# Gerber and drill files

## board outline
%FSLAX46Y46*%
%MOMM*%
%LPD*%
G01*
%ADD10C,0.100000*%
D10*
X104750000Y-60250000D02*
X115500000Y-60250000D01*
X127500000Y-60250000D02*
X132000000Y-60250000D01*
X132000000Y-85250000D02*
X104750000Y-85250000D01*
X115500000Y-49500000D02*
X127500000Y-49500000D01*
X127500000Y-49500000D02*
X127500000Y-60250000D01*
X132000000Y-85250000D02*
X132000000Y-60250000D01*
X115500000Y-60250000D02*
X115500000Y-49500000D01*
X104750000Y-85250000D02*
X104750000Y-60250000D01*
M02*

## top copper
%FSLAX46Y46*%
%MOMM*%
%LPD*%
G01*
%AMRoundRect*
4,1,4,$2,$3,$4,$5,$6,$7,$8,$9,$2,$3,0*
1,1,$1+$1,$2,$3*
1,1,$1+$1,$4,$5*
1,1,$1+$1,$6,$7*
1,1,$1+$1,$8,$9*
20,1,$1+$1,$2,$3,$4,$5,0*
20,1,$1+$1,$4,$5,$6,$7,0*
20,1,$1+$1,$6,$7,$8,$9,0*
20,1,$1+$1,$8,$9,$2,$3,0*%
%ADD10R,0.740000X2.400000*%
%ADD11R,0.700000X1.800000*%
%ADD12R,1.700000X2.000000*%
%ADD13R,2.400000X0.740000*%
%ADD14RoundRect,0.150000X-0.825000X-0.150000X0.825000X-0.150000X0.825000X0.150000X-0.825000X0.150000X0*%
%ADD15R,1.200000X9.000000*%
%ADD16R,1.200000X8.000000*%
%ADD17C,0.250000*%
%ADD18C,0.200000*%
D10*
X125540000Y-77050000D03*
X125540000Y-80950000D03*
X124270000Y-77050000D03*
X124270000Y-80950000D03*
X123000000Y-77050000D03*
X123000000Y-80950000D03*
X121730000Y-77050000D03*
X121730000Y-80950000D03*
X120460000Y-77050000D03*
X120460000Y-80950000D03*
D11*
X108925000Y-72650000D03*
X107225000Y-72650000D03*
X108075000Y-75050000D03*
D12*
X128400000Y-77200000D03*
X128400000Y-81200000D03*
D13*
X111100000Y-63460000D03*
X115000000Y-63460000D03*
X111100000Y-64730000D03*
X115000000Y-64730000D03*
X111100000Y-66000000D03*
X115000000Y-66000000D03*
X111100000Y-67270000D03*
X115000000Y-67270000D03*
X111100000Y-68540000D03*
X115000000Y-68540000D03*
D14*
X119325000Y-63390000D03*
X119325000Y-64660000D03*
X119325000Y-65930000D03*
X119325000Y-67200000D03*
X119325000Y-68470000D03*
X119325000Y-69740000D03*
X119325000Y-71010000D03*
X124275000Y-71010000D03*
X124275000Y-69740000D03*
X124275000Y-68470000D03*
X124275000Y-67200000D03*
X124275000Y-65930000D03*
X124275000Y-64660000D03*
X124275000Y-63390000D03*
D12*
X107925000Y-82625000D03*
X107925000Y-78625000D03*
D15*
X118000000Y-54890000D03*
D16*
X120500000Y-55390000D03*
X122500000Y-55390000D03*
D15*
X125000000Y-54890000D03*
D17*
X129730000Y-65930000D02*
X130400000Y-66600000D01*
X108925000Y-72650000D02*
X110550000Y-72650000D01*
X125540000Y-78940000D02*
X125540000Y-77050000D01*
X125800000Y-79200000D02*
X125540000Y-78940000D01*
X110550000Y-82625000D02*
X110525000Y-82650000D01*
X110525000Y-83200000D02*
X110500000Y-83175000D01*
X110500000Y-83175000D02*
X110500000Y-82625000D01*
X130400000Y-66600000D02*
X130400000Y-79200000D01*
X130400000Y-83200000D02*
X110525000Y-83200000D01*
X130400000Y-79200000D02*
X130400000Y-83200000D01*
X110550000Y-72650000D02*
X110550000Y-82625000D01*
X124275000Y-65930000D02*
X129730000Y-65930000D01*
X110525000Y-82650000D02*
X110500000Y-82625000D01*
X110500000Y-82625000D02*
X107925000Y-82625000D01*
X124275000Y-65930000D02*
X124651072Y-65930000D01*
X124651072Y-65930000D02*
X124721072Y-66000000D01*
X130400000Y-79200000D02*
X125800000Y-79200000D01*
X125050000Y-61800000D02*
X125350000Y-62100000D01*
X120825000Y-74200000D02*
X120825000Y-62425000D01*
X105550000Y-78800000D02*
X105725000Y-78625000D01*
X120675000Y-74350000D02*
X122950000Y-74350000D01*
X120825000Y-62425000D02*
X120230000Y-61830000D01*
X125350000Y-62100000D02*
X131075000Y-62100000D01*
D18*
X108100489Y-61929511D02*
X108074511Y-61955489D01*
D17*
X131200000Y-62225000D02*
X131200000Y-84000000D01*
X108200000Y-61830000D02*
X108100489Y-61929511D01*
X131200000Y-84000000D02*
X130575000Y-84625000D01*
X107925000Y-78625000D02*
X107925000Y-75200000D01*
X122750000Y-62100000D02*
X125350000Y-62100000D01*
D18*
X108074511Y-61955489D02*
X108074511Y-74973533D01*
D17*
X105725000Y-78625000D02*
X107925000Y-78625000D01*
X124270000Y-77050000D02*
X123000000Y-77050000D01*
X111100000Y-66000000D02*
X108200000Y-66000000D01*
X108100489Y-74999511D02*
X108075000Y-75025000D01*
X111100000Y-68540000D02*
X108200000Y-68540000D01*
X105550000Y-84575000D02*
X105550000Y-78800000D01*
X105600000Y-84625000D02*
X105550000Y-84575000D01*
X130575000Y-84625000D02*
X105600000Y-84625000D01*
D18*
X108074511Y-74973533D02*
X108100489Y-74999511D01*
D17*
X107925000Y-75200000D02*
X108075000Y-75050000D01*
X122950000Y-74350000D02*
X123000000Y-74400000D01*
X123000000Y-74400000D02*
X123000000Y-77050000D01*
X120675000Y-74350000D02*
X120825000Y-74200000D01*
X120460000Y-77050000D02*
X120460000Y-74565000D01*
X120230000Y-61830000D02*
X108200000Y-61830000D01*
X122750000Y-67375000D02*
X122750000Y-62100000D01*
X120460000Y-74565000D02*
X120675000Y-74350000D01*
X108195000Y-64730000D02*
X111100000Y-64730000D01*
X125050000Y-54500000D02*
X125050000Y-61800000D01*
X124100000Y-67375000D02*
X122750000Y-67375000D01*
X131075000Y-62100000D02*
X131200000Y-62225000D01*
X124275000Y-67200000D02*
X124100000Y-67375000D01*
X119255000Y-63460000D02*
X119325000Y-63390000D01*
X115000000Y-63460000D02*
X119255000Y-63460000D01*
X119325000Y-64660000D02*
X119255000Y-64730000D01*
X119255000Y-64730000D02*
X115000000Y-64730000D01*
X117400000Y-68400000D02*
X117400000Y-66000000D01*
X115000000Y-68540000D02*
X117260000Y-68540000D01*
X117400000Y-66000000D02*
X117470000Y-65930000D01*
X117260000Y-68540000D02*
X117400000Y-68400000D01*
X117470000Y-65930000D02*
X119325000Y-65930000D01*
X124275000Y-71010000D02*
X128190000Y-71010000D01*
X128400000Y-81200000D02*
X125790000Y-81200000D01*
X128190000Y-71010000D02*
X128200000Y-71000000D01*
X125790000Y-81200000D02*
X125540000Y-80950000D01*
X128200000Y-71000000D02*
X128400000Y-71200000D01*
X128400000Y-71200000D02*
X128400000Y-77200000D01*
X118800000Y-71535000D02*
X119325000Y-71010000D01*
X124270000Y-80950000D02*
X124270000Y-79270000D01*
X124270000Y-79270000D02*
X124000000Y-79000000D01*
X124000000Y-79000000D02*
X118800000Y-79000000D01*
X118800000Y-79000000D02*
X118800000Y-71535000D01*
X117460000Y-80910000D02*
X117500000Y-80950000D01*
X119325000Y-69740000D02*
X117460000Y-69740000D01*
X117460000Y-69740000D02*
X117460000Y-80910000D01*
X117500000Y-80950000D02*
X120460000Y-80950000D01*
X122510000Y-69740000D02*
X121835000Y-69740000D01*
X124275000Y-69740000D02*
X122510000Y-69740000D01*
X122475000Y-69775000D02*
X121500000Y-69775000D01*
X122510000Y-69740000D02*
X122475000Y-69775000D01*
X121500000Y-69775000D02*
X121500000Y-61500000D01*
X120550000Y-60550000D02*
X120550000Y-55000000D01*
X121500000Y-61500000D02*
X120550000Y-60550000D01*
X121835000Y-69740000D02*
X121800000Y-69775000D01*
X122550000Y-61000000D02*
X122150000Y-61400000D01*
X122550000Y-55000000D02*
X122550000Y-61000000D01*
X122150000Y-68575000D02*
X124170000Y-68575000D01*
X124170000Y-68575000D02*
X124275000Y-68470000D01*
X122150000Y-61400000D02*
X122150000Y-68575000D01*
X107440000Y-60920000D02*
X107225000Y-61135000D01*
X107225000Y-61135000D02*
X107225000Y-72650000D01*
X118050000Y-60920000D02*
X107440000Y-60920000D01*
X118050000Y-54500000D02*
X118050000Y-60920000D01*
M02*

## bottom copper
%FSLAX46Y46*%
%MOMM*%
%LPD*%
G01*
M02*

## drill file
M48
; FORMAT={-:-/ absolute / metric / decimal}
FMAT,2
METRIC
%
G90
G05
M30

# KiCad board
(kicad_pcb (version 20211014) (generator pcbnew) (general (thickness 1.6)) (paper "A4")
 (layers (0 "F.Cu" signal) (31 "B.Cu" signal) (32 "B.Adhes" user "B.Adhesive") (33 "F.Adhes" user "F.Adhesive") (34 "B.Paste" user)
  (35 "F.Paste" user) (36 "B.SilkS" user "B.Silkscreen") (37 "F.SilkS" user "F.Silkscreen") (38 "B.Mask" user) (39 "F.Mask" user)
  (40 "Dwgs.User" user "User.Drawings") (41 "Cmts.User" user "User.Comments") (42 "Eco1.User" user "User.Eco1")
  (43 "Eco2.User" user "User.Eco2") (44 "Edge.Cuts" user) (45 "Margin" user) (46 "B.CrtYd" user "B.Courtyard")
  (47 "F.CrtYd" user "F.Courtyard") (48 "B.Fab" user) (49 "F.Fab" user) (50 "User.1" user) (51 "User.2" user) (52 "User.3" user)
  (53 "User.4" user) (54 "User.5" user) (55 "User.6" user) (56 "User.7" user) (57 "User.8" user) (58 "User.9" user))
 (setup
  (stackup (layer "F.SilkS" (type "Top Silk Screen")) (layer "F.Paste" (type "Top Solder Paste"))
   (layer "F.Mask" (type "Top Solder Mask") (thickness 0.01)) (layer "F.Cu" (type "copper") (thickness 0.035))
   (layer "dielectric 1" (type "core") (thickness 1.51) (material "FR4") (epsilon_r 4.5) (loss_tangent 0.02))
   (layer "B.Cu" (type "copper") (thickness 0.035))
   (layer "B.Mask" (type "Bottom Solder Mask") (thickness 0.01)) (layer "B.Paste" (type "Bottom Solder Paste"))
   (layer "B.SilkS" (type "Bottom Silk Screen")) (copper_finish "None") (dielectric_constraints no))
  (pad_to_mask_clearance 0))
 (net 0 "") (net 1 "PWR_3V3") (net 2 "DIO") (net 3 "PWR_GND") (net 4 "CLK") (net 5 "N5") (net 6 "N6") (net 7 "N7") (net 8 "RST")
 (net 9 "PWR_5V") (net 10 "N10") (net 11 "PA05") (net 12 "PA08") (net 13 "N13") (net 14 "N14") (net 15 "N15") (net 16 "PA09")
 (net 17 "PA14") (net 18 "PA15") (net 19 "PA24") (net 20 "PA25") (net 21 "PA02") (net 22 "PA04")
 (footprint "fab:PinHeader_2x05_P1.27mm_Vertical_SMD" (layer "F.Cu") (at 123 79 -90)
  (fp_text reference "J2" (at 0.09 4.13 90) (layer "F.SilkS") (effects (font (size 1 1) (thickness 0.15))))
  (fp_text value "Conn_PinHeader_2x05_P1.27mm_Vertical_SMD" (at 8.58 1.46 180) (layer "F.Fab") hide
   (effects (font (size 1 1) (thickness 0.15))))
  (pad "1" smd rect locked (at -1.95 -2.54 270) (size 2.4 0.74) (layers "F.Cu" "F.Paste" "F.Mask") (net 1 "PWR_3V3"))
  (pad "2" smd rect locked (at 1.95 -2.54 270) (size 2.4 0.74) (layers "F.Cu" "F.Paste" "F.Mask") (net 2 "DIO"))
  (pad "3" smd rect locked (at -1.95 -1.27 270) (size 2.4 0.74) (layers "F.Cu" "F.Paste" "F.Mask") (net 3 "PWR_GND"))
  (pad "4" smd rect locked (at 1.95 -1.27 270) (size 2.4 0.74) (layers "F.Cu" "F.Paste" "F.Mask") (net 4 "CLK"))
  (pad "5" smd rect locked (at -1.95 0 270) (size 2.4 0.74) (layers "F.Cu" "F.Paste" "F.Mask") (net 3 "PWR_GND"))
  (pad "6" smd rect locked (at 1.95 0 270) (size 2.4 0.74) (layers "F.Cu" "F.Paste" "F.Mask") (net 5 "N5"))
  (pad "7" smd rect locked (at -1.95 1.27 270) (size 2.4 0.74) (layers "F.Cu" "F.Paste" "F.Mask") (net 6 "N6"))
  (pad "8" smd rect locked (at 1.95 1.27 270) (size 2.4 0.74) (layers "F.Cu" "F.Paste" "F.Mask") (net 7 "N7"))
  (pad "9" smd rect locked (at -1.95 2.54 270) (size 2.4 0.74) (layers "F.Cu" "F.Paste" "F.Mask") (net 3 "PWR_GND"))
  (pad "10" smd rect locked (at 1.95 2.54 270) (size 2.4 0.74) (layers "F.Cu" "F.Paste" "F.Mask") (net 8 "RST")))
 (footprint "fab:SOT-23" (layer "F.Cu") (at 108.075 73.85 -90)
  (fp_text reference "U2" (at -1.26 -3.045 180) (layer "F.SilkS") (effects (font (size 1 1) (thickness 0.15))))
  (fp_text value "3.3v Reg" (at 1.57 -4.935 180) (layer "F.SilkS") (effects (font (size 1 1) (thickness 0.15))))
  (pad "1" smd rect (at -1.2 -0.85 270) (size 1.8 0.7) (layers "F.Cu" "F.Paste" "F.Mask") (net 1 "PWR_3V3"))
  (pad "2" smd rect (at -1.2 0.85 270) (size 1.8 0.7) (layers "F.Cu" "F.Paste" "F.Mask") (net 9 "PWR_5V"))
  (pad "3" smd rect (at 1.2 0 270) (size 1.8 0.7) (layers "F.Cu" "F.Paste" "F.Mask") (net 3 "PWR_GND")))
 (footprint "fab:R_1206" (layer "F.Cu") (at 128.4 79.2 -90)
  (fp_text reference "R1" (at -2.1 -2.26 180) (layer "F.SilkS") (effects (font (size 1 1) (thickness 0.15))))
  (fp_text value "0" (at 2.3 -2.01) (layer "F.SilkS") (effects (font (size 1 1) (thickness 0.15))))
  (pad "1" smd rect locked (at -2 0 270) (size 2 1.7) (layers "F.Cu" "F.Paste" "F.Mask") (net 2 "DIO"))
  (pad "2" smd rect locked (at 2 0 270) (size 2 1.7) (layers "F.Cu" "F.Paste" "F.Mask") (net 2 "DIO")))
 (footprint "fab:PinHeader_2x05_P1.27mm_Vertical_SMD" (layer "F.Cu") (at 113.05 66)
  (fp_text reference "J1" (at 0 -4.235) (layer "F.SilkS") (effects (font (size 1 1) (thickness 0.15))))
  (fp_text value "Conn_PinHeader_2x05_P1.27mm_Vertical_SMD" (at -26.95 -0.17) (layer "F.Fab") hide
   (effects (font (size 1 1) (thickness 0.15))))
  (pad "1" smd rect locked (at -1.95 -2.54) (size 2.4 0.74) (layers "F.Cu" "F.Paste" "F.Mask") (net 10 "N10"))
  (pad "2" smd rect locked (at 1.95 -2.54) (size 2.4 0.74) (layers "F.Cu" "F.Paste" "F.Mask") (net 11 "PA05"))
  (pad "3" smd rect locked (at -1.95 -1.27) (size 2.4 0.74) (layers "F.Cu" "F.Paste" "F.Mask") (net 3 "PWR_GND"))
  (pad "4" smd rect locked (at 1.95 -1.27) (size 2.4 0.74) (layers "F.Cu" "F.Paste" "F.Mask") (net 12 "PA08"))
  (pad "5" smd rect locked (at -1.95 0) (size 2.4 0.74) (layers "F.Cu" "F.Paste" "F.Mask") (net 3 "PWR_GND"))
  (pad "6" smd rect locked (at 1.95 0) (size 2.4 0.74) (layers "F.Cu" "F.Paste" "F.Mask") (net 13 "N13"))
  (pad "7" smd rect locked (at -1.95 1.27) (size 2.4 0.74) (layers "F.Cu" "F.Paste" "F.Mask") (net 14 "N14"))
  (pad "8" smd rect locked (at 1.95 1.27) (size 2.4 0.74) (layers "F.Cu" "F.Paste" "F.Mask") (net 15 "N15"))
  (pad "9" smd rect locked (at -1.95 2.54) (size 2.4 0.74) (layers "F.Cu" "F.Paste" "F.Mask") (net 3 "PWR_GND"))
  (pad "10" smd rect locked (at 1.95 2.54) (size 2.4 0.74) (layers "F.Cu" "F.Paste" "F.Mask") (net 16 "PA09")))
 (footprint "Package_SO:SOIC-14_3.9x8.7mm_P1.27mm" (layer "F.Cu") (at 121.8 67.2)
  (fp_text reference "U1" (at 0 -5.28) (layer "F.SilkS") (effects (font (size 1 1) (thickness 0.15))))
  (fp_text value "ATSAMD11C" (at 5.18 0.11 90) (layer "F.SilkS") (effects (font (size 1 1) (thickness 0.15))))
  (pad "1" smd roundrect (at -2.475 -3.81) (size 1.95 0.6) (layers "F.Cu" "F.Paste" "F.Mask") (roundrect_rratio 0.25) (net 11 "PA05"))
  (pad "2" smd roundrect (at -2.475 -2.54) (size 1.95 0.6) (layers "F.Cu" "F.Paste" "F.Mask") (roundrect_rratio 0.25) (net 12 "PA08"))
  (pad "3" smd roundrect (at -2.475 -1.27) (size 1.95 0.6) (layers "F.Cu" "F.Paste" "F.Mask") (roundrect_rratio 0.25) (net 16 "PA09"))
  (pad "4" smd roundrect (at -2.475 0) (size 1.95 0.6) (layers "F.Cu" "F.Paste" "F.Mask") (roundrect_rratio 0.25) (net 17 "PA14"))
  (pad "5" smd roundrect (at -2.475 1.27) (size 1.95 0.6) (layers "F.Cu" "F.Paste" "F.Mask") (roundrect_rratio 0.25) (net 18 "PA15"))
  (pad "6" smd roundrect (at -2.475 2.54) (size 1.95 0.6) (layers "F.Cu" "F.Paste" "F.Mask") (roundrect_rratio 0.25) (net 8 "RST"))
  (pad "7" smd roundrect (at -2.475 3.81) (size 1.95 0.6) (layers "F.Cu" "F.Paste" "F.Mask") (roundrect_rratio 0.25) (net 4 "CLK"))
  (pad "8" smd roundrect (at 2.475 3.81) (size 1.95 0.6) (layers "F.Cu" "F.Paste" "F.Mask") (roundrect_rratio 0.25) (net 2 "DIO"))
  (pad "9" smd roundrect (at 2.475 2.54) (size 1.95 0.6) (layers "F.Cu" "F.Paste" "F.Mask") (roundrect_rratio 0.25) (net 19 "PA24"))
  (pad "10" smd roundrect (at 2.475 1.27) (size 1.95 0.6) (layers "F.Cu" "F.Paste" "F.Mask") (roundrect_rratio 0.25) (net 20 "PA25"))
  (pad "11" smd roundrect (at 2.475 0) (size 1.95 0.6) (layers "F.Cu" "F.Paste" "F.Mask") (roundrect_rratio 0.25) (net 3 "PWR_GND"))
  (pad "12" smd roundrect (at 2.475 -1.27) (size 1.95 0.6) (layers "F.Cu" "F.Paste" "F.Mask") (roundrect_rratio 0.25) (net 1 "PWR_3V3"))
  (pad "13" smd roundrect (at 2.475 -2.54) (size 1.95 0.6) (layers "F.Cu" "F.Paste" "F.Mask") (roundrect_rratio 0.25) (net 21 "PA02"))
  (pad "14" smd roundrect (at 2.475 -3.81) (size 1.95 0.6) (layers "F.Cu" "F.Paste" "F.Mask") (roundrect_rratio 0.25) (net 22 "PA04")))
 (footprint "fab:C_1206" (layer "F.Cu") (at 107.925 80.625 90)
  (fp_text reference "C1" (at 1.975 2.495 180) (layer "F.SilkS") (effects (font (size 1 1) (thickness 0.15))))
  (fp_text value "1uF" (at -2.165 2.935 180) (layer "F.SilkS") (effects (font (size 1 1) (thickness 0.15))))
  (pad "1" smd rect (at -2 0 90) (size 2 1.7) (layers "F.Cu" "F.Paste" "F.Mask") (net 1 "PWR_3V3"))
  (pad "2" smd rect (at 2 0 90) (size 2 1.7) (layers "F.Cu" "F.Paste" "F.Mask") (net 3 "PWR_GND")))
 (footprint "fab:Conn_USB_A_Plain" (layer "F.Cu") (at 121.5 54.89 90)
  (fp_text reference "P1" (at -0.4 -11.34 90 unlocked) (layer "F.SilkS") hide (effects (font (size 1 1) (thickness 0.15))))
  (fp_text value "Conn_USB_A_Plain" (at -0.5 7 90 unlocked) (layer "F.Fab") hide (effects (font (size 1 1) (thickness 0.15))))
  (pad "1" smd rect (at 0 -3.5 90) (size 9 1.2) (layers "F.Cu" "F.Paste" "F.Mask") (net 9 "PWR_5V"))
  (pad "2" smd rect (at -0.5 -1 90) (size 8 1.2) (layers "F.Cu" "F.Paste" "F.Mask") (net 19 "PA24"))
  (pad "3" smd rect (at -0.5 1 90) (size 8 1.2) (layers "F.Cu" "F.Paste" "F.Mask") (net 20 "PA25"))
  (pad "4" smd rect (at 0 3.5 90) (size 9 1.2) (layers "F.Cu" "F.Paste" "F.Mask") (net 3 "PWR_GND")))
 (gr_line (start 104.75 60.25) (end 115.5 60.25) (layer "Edge.Cuts") (width 0.1))
 (gr_line (start 127.5 60.25) (end 132 60.25) (layer "Edge.Cuts") (width 0.1))
 (gr_line (start 132 85.25) (end 104.75 85.25) (layer "Edge.Cuts") (width 0.1))
 (gr_line (start 115.5 49.5) (end 127.5 49.5) (layer "Edge.Cuts") (width 0.1))
 (gr_line (start 127.5 49.5) (end 127.5 60.25) (layer "Edge.Cuts") (width 0.1))
 (gr_line (start 132 85.25) (end 132 60.25) (layer "Edge.Cuts") (width 0.1))
 (gr_line (start 115.5 60.25) (end 115.5 49.5) (layer "Edge.Cuts") (width 0.1))
 (gr_line (start 104.75 85.25) (end 104.75 60.25) (layer "Edge.Cuts") (width 0.1))
 (segment (start 129.73 65.93) (end 130.4 66.6) (width 0.25) (layer "F.Cu") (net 1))
 (segment (start 108.925 72.65) (end 110.55 72.65) (width 0.25) (layer "F.Cu") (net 1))
 (segment (start 125.54 78.94) (end 125.54 77.05) (width 0.25) (layer "F.Cu") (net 1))
 (segment (start 125.8 79.2) (end 125.54 78.94) (width 0.25) (layer "F.Cu") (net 1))
 (segment (start 110.55 82.625) (end 110.525 82.65) (width 0.25) (layer "F.Cu") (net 1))
 (segment (start 110.525 83.2) (end 110.5 83.175) (width 0.25) (layer "F.Cu") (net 1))
 (segment (start 110.5 83.175) (end 110.5 82.625) (width 0.25) (layer "F.Cu") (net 1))
 (segment (start 130.4 66.6) (end 130.4 79.2) (width 0.25) (layer "F.Cu") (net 1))
 (segment (start 130.4 83.2) (end 110.525 83.2) (width 0.25) (layer "F.Cu") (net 1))
 (segment (start 130.4 79.2) (end 130.4 83.2) (width 0.25) (layer "F.Cu") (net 1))
 (segment (start 110.55 72.65) (end 110.55 82.625) (width 0.25) (layer "F.Cu") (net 1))
 (segment (start 124.275 65.93) (end 129.73 65.93) (width 0.25) (layer "F.Cu") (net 1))
 (segment (start 110.525 82.65) (end 110.5 82.625) (width 0.25) (layer "F.Cu") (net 1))
 (segment (start 110.5 82.625) (end 107.925 82.625) (width 0.25) (layer "F.Cu") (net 1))
 (segment (start 124.275 65.93) (end 124.651072 65.93) (width 0.25) (layer "F.Cu") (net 1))
 (segment (start 124.651072 65.93) (end 124.721072 66) (width 0.25) (layer "F.Cu") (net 1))
 (segment (start 130.4 79.2) (end 125.8 79.2) (width 0.25) (layer "F.Cu") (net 1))
 (segment (start 125.05 61.8) (end 125.35 62.1) (width 0.25) (layer "F.Cu") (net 3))
 (segment (start 120.825 74.2) (end 120.825 62.425) (width 0.25) (layer "F.Cu") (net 3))
 (segment (start 105.55 78.8) (end 105.725 78.625) (width 0.25) (layer "F.Cu") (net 3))
 (segment (start 120.675 74.35) (end 122.95 74.35) (width 0.25) (layer "F.Cu") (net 3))
 (segment (start 120.825 62.425) (end 120.23 61.83) (width 0.25) (layer "F.Cu") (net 3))
 (segment (start 125.35 62.1) (end 131.075 62.1) (width 0.25) (layer "F.Cu") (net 3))
 (segment (start 108.100489 61.929511) (end 108.074511 61.955489) (width 0.2) (layer "F.Cu") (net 3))
 (segment (start 131.2 62.225) (end 131.2 84) (width 0.25) (layer "F.Cu") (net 3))
 (segment (start 108.2 61.83) (end 108.100489 61.929511) (width 0.25) (layer "F.Cu") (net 3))
 (segment (start 131.2 84) (end 130.575 84.625) (width 0.25) (layer "F.Cu") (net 3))
 (segment (start 107.925 78.625) (end 107.925 75.2) (width 0.25) (layer "F.Cu") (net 3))
 (segment (start 122.75 62.1) (end 125.35 62.1) (width 0.25) (layer "F.Cu") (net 3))
 (segment (start 108.074511 61.955489) (end 108.074511 74.973533) (width 0.2) (layer "F.Cu") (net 3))
 (segment (start 105.725 78.625) (end 107.925 78.625) (width 0.25) (layer "F.Cu") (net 3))
 (segment (start 124.27 77.05) (end 123 77.05) (width 0.25) (layer "F.Cu") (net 3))
 (segment (start 111.1 66) (end 108.2 66) (width 0.25) (layer "F.Cu") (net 3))
 (segment (start 108.100489 74.999511) (end 108.075 75.025) (width 0.25) (layer "F.Cu") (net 3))
 (segment (start 111.1 68.54) (end 108.2 68.54) (width 0.25) (layer "F.Cu") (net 3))
 (segment (start 105.55 84.575) (end 105.55 78.8) (width 0.25) (layer "F.Cu") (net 3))
 (segment (start 105.6 84.625) (end 105.55 84.575) (width 0.25) (layer "F.Cu") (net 3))
 (segment (start 130.575 84.625) (end 105.6 84.625) (width 0.25) (layer "F.Cu") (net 3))
 (segment (start 108.074511 74.973533) (end 108.100489 74.999511) (width 0.2) (layer "F.Cu") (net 3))
 (segment (start 107.925 75.2) (end 108.075 75.05) (width 0.25) (layer "F.Cu") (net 3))
 (segment (start 122.95 74.35) (end 123 74.4) (width 0.25) (layer "F.Cu") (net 3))
 (segment (start 123 74.4) (end 123 77.05) (width 0.25) (layer "F.Cu") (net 3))
 (segment (start 120.675 74.35) (end 120.825 74.2) (width 0.25) (layer "F.Cu") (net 3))
 (segment (start 120.46 77.05) (end 120.46 74.565) (width 0.25) (layer "F.Cu") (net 3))
 (segment (start 120.23 61.83) (end 108.2 61.83) (width 0.25) (layer "F.Cu") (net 3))
 (segment (start 122.75 67.375) (end 122.75 62.1) (width 0.25) (layer "F.Cu") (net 3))
 (segment (start 120.46 74.565) (end 120.675 74.35) (width 0.25) (layer "F.Cu") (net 3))
 (segment (start 108.195 64.73) (end 111.1 64.73) (width 0.25) (layer "F.Cu") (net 3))
 (segment (start 125.05 54.5) (end 125.05 61.8) (width 0.25) (layer "F.Cu") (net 3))
 (segment (start 124.1 67.375) (end 122.75 67.375) (width 0.25) (layer "F.Cu") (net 3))
 (segment (start 131.075 62.1) (end 131.2 62.225) (width 0.25) (layer "F.Cu") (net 3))
 (segment (start 124.275 67.2) (end 124.1 67.375) (width 0.25) (layer "F.Cu") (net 3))
 (segment (start 119.255 63.46) (end 119.325 63.39) (width 0.25) (layer "F.Cu") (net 11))
 (segment (start 115 63.46) (end 119.255 63.46) (width 0.25) (layer "F.Cu") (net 11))
 (segment (start 119.325 64.66) (end 119.255 64.73) (width 0.25) (layer "F.Cu") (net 12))
 (segment (start 119.255 64.73) (end 115 64.73) (width 0.25) (layer "F.Cu") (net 12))
 (segment (start 117.4 68.4) (end 117.4 66) (width 0.25) (layer "F.Cu") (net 16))
 (segment (start 115 68.54) (end 117.26 68.54) (width 0.25) (layer "F.Cu") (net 16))
 (segment (start 117.4 66) (end 117.47 65.93) (width 0.25) (layer "F.Cu") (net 16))
 (segment (start 117.26 68.54) (end 117.4 68.4) (width 0.25) (layer "F.Cu") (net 16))
 (segment (start 117.47 65.93) (end 119.325 65.93) (width 0.25) (layer "F.Cu") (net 16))
 (segment (start 124.275 71.01) (end 128.19 71.01) (width 0.25) (layer "F.Cu") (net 2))
 (segment (start 128.4 81.2) (end 125.79 81.2) (width 0.25) (layer "F.Cu") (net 2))
 (segment (start 128.19 71.01) (end 128.2 71) (width 0.25) (layer "F.Cu") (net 2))
 (segment (start 125.79 81.2) (end 125.54 80.95) (width 0.25) (layer "F.Cu") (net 2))
 (segment (start 128.2 71) (end 128.4 71.2) (width 0.25) (layer "F.Cu") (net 2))
 (segment (start 128.4 71.2) (end 128.4 77.2) (width 0.25) (layer "F.Cu") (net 2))
 (segment (start 118.8 71.535) (end 119.325 71.01) (width 0.25) (layer "F.Cu") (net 4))
 (segment (start 124.27 80.95) (end 124.27 79.27) (width 0.25) (layer "F.Cu") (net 4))
 (segment (start 124.27 79.27) (end 124 79) (width 0.25) (layer "F.Cu") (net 4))
 (segment (start 124 79) (end 118.8 79) (width 0.25) (layer "F.Cu") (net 4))
 (segment (start 118.8 79) (end 118.8 71.535) (width 0.25) (layer "F.Cu") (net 4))
 (segment (start 117.46 80.91) (end 117.5 80.95) (width 0.25) (layer "F.Cu") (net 8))
 (segment (start 119.325 69.74) (end 117.46 69.74) (width 0.25) (layer "F.Cu") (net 8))
 (segment (start 117.46 69.74) (end 117.46 80.91) (width 0.25) (layer "F.Cu") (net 8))
 (segment (start 117.5 80.95) (end 120.46 80.95) (width 0.25) (layer "F.Cu") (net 8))
 (segment (start 122.51 69.74) (end 121.835 69.74) (width 0.25) (layer "F.Cu") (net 19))
 (segment (start 124.275 69.74) (end 122.51 69.74) (width 0.25) (layer "F.Cu") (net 19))
 (segment (start 122.475 69.775) (end 121.5 69.775) (width 0.25) (layer "F.Cu") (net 19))
 (segment (start 122.51 69.74) (end 122.475 69.775) (width 0.25) (layer "F.Cu") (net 19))
 (segment (start 121.5 69.775) (end 121.5 61.5) (width 0.25) (layer "F.Cu") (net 19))
 (segment (start 120.55 60.55) (end 120.55 55) (width 0.25) (layer "F.Cu") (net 19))
 (segment (start 121.5 61.5) (end 120.55 60.55) (width 0.25) (layer "F.Cu") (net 19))
 (segment (start 121.835 69.74) (end 121.8 69.775) (width 0.25) (layer "F.Cu") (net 19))
 (segment (start 122.55 61) (end 122.15 61.4) (width 0.25) (layer "F.Cu") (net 20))
 (segment (start 122.55 55) (end 122.55 61) (width 0.25) (layer "F.Cu") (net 20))
 (segment (start 122.15 68.575) (end 124.17 68.575) (width 0.25) (layer "F.Cu") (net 20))
 (segment (start 124.17 68.575) (end 124.275 68.47) (width 0.25) (layer "F.Cu") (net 20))
 (segment (start 122.15 61.4) (end 122.15 68.575) (width 0.25) (layer "F.Cu") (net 20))
 (segment (start 107.44 60.92) (end 107.225 61.135) (width 0.25) (layer "F.Cu") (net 9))
 (segment (start 107.225 61.135) (end 107.225 72.65) (width 0.25) (layer "F.Cu") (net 9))
 (segment (start 118.05 60.92) (end 107.44 60.92) (width 0.25) (layer "F.Cu") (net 9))
 (segment (start 118.05 54.5) (end 118.05 60.92) (width 0.25) (layer "F.Cu") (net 9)))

